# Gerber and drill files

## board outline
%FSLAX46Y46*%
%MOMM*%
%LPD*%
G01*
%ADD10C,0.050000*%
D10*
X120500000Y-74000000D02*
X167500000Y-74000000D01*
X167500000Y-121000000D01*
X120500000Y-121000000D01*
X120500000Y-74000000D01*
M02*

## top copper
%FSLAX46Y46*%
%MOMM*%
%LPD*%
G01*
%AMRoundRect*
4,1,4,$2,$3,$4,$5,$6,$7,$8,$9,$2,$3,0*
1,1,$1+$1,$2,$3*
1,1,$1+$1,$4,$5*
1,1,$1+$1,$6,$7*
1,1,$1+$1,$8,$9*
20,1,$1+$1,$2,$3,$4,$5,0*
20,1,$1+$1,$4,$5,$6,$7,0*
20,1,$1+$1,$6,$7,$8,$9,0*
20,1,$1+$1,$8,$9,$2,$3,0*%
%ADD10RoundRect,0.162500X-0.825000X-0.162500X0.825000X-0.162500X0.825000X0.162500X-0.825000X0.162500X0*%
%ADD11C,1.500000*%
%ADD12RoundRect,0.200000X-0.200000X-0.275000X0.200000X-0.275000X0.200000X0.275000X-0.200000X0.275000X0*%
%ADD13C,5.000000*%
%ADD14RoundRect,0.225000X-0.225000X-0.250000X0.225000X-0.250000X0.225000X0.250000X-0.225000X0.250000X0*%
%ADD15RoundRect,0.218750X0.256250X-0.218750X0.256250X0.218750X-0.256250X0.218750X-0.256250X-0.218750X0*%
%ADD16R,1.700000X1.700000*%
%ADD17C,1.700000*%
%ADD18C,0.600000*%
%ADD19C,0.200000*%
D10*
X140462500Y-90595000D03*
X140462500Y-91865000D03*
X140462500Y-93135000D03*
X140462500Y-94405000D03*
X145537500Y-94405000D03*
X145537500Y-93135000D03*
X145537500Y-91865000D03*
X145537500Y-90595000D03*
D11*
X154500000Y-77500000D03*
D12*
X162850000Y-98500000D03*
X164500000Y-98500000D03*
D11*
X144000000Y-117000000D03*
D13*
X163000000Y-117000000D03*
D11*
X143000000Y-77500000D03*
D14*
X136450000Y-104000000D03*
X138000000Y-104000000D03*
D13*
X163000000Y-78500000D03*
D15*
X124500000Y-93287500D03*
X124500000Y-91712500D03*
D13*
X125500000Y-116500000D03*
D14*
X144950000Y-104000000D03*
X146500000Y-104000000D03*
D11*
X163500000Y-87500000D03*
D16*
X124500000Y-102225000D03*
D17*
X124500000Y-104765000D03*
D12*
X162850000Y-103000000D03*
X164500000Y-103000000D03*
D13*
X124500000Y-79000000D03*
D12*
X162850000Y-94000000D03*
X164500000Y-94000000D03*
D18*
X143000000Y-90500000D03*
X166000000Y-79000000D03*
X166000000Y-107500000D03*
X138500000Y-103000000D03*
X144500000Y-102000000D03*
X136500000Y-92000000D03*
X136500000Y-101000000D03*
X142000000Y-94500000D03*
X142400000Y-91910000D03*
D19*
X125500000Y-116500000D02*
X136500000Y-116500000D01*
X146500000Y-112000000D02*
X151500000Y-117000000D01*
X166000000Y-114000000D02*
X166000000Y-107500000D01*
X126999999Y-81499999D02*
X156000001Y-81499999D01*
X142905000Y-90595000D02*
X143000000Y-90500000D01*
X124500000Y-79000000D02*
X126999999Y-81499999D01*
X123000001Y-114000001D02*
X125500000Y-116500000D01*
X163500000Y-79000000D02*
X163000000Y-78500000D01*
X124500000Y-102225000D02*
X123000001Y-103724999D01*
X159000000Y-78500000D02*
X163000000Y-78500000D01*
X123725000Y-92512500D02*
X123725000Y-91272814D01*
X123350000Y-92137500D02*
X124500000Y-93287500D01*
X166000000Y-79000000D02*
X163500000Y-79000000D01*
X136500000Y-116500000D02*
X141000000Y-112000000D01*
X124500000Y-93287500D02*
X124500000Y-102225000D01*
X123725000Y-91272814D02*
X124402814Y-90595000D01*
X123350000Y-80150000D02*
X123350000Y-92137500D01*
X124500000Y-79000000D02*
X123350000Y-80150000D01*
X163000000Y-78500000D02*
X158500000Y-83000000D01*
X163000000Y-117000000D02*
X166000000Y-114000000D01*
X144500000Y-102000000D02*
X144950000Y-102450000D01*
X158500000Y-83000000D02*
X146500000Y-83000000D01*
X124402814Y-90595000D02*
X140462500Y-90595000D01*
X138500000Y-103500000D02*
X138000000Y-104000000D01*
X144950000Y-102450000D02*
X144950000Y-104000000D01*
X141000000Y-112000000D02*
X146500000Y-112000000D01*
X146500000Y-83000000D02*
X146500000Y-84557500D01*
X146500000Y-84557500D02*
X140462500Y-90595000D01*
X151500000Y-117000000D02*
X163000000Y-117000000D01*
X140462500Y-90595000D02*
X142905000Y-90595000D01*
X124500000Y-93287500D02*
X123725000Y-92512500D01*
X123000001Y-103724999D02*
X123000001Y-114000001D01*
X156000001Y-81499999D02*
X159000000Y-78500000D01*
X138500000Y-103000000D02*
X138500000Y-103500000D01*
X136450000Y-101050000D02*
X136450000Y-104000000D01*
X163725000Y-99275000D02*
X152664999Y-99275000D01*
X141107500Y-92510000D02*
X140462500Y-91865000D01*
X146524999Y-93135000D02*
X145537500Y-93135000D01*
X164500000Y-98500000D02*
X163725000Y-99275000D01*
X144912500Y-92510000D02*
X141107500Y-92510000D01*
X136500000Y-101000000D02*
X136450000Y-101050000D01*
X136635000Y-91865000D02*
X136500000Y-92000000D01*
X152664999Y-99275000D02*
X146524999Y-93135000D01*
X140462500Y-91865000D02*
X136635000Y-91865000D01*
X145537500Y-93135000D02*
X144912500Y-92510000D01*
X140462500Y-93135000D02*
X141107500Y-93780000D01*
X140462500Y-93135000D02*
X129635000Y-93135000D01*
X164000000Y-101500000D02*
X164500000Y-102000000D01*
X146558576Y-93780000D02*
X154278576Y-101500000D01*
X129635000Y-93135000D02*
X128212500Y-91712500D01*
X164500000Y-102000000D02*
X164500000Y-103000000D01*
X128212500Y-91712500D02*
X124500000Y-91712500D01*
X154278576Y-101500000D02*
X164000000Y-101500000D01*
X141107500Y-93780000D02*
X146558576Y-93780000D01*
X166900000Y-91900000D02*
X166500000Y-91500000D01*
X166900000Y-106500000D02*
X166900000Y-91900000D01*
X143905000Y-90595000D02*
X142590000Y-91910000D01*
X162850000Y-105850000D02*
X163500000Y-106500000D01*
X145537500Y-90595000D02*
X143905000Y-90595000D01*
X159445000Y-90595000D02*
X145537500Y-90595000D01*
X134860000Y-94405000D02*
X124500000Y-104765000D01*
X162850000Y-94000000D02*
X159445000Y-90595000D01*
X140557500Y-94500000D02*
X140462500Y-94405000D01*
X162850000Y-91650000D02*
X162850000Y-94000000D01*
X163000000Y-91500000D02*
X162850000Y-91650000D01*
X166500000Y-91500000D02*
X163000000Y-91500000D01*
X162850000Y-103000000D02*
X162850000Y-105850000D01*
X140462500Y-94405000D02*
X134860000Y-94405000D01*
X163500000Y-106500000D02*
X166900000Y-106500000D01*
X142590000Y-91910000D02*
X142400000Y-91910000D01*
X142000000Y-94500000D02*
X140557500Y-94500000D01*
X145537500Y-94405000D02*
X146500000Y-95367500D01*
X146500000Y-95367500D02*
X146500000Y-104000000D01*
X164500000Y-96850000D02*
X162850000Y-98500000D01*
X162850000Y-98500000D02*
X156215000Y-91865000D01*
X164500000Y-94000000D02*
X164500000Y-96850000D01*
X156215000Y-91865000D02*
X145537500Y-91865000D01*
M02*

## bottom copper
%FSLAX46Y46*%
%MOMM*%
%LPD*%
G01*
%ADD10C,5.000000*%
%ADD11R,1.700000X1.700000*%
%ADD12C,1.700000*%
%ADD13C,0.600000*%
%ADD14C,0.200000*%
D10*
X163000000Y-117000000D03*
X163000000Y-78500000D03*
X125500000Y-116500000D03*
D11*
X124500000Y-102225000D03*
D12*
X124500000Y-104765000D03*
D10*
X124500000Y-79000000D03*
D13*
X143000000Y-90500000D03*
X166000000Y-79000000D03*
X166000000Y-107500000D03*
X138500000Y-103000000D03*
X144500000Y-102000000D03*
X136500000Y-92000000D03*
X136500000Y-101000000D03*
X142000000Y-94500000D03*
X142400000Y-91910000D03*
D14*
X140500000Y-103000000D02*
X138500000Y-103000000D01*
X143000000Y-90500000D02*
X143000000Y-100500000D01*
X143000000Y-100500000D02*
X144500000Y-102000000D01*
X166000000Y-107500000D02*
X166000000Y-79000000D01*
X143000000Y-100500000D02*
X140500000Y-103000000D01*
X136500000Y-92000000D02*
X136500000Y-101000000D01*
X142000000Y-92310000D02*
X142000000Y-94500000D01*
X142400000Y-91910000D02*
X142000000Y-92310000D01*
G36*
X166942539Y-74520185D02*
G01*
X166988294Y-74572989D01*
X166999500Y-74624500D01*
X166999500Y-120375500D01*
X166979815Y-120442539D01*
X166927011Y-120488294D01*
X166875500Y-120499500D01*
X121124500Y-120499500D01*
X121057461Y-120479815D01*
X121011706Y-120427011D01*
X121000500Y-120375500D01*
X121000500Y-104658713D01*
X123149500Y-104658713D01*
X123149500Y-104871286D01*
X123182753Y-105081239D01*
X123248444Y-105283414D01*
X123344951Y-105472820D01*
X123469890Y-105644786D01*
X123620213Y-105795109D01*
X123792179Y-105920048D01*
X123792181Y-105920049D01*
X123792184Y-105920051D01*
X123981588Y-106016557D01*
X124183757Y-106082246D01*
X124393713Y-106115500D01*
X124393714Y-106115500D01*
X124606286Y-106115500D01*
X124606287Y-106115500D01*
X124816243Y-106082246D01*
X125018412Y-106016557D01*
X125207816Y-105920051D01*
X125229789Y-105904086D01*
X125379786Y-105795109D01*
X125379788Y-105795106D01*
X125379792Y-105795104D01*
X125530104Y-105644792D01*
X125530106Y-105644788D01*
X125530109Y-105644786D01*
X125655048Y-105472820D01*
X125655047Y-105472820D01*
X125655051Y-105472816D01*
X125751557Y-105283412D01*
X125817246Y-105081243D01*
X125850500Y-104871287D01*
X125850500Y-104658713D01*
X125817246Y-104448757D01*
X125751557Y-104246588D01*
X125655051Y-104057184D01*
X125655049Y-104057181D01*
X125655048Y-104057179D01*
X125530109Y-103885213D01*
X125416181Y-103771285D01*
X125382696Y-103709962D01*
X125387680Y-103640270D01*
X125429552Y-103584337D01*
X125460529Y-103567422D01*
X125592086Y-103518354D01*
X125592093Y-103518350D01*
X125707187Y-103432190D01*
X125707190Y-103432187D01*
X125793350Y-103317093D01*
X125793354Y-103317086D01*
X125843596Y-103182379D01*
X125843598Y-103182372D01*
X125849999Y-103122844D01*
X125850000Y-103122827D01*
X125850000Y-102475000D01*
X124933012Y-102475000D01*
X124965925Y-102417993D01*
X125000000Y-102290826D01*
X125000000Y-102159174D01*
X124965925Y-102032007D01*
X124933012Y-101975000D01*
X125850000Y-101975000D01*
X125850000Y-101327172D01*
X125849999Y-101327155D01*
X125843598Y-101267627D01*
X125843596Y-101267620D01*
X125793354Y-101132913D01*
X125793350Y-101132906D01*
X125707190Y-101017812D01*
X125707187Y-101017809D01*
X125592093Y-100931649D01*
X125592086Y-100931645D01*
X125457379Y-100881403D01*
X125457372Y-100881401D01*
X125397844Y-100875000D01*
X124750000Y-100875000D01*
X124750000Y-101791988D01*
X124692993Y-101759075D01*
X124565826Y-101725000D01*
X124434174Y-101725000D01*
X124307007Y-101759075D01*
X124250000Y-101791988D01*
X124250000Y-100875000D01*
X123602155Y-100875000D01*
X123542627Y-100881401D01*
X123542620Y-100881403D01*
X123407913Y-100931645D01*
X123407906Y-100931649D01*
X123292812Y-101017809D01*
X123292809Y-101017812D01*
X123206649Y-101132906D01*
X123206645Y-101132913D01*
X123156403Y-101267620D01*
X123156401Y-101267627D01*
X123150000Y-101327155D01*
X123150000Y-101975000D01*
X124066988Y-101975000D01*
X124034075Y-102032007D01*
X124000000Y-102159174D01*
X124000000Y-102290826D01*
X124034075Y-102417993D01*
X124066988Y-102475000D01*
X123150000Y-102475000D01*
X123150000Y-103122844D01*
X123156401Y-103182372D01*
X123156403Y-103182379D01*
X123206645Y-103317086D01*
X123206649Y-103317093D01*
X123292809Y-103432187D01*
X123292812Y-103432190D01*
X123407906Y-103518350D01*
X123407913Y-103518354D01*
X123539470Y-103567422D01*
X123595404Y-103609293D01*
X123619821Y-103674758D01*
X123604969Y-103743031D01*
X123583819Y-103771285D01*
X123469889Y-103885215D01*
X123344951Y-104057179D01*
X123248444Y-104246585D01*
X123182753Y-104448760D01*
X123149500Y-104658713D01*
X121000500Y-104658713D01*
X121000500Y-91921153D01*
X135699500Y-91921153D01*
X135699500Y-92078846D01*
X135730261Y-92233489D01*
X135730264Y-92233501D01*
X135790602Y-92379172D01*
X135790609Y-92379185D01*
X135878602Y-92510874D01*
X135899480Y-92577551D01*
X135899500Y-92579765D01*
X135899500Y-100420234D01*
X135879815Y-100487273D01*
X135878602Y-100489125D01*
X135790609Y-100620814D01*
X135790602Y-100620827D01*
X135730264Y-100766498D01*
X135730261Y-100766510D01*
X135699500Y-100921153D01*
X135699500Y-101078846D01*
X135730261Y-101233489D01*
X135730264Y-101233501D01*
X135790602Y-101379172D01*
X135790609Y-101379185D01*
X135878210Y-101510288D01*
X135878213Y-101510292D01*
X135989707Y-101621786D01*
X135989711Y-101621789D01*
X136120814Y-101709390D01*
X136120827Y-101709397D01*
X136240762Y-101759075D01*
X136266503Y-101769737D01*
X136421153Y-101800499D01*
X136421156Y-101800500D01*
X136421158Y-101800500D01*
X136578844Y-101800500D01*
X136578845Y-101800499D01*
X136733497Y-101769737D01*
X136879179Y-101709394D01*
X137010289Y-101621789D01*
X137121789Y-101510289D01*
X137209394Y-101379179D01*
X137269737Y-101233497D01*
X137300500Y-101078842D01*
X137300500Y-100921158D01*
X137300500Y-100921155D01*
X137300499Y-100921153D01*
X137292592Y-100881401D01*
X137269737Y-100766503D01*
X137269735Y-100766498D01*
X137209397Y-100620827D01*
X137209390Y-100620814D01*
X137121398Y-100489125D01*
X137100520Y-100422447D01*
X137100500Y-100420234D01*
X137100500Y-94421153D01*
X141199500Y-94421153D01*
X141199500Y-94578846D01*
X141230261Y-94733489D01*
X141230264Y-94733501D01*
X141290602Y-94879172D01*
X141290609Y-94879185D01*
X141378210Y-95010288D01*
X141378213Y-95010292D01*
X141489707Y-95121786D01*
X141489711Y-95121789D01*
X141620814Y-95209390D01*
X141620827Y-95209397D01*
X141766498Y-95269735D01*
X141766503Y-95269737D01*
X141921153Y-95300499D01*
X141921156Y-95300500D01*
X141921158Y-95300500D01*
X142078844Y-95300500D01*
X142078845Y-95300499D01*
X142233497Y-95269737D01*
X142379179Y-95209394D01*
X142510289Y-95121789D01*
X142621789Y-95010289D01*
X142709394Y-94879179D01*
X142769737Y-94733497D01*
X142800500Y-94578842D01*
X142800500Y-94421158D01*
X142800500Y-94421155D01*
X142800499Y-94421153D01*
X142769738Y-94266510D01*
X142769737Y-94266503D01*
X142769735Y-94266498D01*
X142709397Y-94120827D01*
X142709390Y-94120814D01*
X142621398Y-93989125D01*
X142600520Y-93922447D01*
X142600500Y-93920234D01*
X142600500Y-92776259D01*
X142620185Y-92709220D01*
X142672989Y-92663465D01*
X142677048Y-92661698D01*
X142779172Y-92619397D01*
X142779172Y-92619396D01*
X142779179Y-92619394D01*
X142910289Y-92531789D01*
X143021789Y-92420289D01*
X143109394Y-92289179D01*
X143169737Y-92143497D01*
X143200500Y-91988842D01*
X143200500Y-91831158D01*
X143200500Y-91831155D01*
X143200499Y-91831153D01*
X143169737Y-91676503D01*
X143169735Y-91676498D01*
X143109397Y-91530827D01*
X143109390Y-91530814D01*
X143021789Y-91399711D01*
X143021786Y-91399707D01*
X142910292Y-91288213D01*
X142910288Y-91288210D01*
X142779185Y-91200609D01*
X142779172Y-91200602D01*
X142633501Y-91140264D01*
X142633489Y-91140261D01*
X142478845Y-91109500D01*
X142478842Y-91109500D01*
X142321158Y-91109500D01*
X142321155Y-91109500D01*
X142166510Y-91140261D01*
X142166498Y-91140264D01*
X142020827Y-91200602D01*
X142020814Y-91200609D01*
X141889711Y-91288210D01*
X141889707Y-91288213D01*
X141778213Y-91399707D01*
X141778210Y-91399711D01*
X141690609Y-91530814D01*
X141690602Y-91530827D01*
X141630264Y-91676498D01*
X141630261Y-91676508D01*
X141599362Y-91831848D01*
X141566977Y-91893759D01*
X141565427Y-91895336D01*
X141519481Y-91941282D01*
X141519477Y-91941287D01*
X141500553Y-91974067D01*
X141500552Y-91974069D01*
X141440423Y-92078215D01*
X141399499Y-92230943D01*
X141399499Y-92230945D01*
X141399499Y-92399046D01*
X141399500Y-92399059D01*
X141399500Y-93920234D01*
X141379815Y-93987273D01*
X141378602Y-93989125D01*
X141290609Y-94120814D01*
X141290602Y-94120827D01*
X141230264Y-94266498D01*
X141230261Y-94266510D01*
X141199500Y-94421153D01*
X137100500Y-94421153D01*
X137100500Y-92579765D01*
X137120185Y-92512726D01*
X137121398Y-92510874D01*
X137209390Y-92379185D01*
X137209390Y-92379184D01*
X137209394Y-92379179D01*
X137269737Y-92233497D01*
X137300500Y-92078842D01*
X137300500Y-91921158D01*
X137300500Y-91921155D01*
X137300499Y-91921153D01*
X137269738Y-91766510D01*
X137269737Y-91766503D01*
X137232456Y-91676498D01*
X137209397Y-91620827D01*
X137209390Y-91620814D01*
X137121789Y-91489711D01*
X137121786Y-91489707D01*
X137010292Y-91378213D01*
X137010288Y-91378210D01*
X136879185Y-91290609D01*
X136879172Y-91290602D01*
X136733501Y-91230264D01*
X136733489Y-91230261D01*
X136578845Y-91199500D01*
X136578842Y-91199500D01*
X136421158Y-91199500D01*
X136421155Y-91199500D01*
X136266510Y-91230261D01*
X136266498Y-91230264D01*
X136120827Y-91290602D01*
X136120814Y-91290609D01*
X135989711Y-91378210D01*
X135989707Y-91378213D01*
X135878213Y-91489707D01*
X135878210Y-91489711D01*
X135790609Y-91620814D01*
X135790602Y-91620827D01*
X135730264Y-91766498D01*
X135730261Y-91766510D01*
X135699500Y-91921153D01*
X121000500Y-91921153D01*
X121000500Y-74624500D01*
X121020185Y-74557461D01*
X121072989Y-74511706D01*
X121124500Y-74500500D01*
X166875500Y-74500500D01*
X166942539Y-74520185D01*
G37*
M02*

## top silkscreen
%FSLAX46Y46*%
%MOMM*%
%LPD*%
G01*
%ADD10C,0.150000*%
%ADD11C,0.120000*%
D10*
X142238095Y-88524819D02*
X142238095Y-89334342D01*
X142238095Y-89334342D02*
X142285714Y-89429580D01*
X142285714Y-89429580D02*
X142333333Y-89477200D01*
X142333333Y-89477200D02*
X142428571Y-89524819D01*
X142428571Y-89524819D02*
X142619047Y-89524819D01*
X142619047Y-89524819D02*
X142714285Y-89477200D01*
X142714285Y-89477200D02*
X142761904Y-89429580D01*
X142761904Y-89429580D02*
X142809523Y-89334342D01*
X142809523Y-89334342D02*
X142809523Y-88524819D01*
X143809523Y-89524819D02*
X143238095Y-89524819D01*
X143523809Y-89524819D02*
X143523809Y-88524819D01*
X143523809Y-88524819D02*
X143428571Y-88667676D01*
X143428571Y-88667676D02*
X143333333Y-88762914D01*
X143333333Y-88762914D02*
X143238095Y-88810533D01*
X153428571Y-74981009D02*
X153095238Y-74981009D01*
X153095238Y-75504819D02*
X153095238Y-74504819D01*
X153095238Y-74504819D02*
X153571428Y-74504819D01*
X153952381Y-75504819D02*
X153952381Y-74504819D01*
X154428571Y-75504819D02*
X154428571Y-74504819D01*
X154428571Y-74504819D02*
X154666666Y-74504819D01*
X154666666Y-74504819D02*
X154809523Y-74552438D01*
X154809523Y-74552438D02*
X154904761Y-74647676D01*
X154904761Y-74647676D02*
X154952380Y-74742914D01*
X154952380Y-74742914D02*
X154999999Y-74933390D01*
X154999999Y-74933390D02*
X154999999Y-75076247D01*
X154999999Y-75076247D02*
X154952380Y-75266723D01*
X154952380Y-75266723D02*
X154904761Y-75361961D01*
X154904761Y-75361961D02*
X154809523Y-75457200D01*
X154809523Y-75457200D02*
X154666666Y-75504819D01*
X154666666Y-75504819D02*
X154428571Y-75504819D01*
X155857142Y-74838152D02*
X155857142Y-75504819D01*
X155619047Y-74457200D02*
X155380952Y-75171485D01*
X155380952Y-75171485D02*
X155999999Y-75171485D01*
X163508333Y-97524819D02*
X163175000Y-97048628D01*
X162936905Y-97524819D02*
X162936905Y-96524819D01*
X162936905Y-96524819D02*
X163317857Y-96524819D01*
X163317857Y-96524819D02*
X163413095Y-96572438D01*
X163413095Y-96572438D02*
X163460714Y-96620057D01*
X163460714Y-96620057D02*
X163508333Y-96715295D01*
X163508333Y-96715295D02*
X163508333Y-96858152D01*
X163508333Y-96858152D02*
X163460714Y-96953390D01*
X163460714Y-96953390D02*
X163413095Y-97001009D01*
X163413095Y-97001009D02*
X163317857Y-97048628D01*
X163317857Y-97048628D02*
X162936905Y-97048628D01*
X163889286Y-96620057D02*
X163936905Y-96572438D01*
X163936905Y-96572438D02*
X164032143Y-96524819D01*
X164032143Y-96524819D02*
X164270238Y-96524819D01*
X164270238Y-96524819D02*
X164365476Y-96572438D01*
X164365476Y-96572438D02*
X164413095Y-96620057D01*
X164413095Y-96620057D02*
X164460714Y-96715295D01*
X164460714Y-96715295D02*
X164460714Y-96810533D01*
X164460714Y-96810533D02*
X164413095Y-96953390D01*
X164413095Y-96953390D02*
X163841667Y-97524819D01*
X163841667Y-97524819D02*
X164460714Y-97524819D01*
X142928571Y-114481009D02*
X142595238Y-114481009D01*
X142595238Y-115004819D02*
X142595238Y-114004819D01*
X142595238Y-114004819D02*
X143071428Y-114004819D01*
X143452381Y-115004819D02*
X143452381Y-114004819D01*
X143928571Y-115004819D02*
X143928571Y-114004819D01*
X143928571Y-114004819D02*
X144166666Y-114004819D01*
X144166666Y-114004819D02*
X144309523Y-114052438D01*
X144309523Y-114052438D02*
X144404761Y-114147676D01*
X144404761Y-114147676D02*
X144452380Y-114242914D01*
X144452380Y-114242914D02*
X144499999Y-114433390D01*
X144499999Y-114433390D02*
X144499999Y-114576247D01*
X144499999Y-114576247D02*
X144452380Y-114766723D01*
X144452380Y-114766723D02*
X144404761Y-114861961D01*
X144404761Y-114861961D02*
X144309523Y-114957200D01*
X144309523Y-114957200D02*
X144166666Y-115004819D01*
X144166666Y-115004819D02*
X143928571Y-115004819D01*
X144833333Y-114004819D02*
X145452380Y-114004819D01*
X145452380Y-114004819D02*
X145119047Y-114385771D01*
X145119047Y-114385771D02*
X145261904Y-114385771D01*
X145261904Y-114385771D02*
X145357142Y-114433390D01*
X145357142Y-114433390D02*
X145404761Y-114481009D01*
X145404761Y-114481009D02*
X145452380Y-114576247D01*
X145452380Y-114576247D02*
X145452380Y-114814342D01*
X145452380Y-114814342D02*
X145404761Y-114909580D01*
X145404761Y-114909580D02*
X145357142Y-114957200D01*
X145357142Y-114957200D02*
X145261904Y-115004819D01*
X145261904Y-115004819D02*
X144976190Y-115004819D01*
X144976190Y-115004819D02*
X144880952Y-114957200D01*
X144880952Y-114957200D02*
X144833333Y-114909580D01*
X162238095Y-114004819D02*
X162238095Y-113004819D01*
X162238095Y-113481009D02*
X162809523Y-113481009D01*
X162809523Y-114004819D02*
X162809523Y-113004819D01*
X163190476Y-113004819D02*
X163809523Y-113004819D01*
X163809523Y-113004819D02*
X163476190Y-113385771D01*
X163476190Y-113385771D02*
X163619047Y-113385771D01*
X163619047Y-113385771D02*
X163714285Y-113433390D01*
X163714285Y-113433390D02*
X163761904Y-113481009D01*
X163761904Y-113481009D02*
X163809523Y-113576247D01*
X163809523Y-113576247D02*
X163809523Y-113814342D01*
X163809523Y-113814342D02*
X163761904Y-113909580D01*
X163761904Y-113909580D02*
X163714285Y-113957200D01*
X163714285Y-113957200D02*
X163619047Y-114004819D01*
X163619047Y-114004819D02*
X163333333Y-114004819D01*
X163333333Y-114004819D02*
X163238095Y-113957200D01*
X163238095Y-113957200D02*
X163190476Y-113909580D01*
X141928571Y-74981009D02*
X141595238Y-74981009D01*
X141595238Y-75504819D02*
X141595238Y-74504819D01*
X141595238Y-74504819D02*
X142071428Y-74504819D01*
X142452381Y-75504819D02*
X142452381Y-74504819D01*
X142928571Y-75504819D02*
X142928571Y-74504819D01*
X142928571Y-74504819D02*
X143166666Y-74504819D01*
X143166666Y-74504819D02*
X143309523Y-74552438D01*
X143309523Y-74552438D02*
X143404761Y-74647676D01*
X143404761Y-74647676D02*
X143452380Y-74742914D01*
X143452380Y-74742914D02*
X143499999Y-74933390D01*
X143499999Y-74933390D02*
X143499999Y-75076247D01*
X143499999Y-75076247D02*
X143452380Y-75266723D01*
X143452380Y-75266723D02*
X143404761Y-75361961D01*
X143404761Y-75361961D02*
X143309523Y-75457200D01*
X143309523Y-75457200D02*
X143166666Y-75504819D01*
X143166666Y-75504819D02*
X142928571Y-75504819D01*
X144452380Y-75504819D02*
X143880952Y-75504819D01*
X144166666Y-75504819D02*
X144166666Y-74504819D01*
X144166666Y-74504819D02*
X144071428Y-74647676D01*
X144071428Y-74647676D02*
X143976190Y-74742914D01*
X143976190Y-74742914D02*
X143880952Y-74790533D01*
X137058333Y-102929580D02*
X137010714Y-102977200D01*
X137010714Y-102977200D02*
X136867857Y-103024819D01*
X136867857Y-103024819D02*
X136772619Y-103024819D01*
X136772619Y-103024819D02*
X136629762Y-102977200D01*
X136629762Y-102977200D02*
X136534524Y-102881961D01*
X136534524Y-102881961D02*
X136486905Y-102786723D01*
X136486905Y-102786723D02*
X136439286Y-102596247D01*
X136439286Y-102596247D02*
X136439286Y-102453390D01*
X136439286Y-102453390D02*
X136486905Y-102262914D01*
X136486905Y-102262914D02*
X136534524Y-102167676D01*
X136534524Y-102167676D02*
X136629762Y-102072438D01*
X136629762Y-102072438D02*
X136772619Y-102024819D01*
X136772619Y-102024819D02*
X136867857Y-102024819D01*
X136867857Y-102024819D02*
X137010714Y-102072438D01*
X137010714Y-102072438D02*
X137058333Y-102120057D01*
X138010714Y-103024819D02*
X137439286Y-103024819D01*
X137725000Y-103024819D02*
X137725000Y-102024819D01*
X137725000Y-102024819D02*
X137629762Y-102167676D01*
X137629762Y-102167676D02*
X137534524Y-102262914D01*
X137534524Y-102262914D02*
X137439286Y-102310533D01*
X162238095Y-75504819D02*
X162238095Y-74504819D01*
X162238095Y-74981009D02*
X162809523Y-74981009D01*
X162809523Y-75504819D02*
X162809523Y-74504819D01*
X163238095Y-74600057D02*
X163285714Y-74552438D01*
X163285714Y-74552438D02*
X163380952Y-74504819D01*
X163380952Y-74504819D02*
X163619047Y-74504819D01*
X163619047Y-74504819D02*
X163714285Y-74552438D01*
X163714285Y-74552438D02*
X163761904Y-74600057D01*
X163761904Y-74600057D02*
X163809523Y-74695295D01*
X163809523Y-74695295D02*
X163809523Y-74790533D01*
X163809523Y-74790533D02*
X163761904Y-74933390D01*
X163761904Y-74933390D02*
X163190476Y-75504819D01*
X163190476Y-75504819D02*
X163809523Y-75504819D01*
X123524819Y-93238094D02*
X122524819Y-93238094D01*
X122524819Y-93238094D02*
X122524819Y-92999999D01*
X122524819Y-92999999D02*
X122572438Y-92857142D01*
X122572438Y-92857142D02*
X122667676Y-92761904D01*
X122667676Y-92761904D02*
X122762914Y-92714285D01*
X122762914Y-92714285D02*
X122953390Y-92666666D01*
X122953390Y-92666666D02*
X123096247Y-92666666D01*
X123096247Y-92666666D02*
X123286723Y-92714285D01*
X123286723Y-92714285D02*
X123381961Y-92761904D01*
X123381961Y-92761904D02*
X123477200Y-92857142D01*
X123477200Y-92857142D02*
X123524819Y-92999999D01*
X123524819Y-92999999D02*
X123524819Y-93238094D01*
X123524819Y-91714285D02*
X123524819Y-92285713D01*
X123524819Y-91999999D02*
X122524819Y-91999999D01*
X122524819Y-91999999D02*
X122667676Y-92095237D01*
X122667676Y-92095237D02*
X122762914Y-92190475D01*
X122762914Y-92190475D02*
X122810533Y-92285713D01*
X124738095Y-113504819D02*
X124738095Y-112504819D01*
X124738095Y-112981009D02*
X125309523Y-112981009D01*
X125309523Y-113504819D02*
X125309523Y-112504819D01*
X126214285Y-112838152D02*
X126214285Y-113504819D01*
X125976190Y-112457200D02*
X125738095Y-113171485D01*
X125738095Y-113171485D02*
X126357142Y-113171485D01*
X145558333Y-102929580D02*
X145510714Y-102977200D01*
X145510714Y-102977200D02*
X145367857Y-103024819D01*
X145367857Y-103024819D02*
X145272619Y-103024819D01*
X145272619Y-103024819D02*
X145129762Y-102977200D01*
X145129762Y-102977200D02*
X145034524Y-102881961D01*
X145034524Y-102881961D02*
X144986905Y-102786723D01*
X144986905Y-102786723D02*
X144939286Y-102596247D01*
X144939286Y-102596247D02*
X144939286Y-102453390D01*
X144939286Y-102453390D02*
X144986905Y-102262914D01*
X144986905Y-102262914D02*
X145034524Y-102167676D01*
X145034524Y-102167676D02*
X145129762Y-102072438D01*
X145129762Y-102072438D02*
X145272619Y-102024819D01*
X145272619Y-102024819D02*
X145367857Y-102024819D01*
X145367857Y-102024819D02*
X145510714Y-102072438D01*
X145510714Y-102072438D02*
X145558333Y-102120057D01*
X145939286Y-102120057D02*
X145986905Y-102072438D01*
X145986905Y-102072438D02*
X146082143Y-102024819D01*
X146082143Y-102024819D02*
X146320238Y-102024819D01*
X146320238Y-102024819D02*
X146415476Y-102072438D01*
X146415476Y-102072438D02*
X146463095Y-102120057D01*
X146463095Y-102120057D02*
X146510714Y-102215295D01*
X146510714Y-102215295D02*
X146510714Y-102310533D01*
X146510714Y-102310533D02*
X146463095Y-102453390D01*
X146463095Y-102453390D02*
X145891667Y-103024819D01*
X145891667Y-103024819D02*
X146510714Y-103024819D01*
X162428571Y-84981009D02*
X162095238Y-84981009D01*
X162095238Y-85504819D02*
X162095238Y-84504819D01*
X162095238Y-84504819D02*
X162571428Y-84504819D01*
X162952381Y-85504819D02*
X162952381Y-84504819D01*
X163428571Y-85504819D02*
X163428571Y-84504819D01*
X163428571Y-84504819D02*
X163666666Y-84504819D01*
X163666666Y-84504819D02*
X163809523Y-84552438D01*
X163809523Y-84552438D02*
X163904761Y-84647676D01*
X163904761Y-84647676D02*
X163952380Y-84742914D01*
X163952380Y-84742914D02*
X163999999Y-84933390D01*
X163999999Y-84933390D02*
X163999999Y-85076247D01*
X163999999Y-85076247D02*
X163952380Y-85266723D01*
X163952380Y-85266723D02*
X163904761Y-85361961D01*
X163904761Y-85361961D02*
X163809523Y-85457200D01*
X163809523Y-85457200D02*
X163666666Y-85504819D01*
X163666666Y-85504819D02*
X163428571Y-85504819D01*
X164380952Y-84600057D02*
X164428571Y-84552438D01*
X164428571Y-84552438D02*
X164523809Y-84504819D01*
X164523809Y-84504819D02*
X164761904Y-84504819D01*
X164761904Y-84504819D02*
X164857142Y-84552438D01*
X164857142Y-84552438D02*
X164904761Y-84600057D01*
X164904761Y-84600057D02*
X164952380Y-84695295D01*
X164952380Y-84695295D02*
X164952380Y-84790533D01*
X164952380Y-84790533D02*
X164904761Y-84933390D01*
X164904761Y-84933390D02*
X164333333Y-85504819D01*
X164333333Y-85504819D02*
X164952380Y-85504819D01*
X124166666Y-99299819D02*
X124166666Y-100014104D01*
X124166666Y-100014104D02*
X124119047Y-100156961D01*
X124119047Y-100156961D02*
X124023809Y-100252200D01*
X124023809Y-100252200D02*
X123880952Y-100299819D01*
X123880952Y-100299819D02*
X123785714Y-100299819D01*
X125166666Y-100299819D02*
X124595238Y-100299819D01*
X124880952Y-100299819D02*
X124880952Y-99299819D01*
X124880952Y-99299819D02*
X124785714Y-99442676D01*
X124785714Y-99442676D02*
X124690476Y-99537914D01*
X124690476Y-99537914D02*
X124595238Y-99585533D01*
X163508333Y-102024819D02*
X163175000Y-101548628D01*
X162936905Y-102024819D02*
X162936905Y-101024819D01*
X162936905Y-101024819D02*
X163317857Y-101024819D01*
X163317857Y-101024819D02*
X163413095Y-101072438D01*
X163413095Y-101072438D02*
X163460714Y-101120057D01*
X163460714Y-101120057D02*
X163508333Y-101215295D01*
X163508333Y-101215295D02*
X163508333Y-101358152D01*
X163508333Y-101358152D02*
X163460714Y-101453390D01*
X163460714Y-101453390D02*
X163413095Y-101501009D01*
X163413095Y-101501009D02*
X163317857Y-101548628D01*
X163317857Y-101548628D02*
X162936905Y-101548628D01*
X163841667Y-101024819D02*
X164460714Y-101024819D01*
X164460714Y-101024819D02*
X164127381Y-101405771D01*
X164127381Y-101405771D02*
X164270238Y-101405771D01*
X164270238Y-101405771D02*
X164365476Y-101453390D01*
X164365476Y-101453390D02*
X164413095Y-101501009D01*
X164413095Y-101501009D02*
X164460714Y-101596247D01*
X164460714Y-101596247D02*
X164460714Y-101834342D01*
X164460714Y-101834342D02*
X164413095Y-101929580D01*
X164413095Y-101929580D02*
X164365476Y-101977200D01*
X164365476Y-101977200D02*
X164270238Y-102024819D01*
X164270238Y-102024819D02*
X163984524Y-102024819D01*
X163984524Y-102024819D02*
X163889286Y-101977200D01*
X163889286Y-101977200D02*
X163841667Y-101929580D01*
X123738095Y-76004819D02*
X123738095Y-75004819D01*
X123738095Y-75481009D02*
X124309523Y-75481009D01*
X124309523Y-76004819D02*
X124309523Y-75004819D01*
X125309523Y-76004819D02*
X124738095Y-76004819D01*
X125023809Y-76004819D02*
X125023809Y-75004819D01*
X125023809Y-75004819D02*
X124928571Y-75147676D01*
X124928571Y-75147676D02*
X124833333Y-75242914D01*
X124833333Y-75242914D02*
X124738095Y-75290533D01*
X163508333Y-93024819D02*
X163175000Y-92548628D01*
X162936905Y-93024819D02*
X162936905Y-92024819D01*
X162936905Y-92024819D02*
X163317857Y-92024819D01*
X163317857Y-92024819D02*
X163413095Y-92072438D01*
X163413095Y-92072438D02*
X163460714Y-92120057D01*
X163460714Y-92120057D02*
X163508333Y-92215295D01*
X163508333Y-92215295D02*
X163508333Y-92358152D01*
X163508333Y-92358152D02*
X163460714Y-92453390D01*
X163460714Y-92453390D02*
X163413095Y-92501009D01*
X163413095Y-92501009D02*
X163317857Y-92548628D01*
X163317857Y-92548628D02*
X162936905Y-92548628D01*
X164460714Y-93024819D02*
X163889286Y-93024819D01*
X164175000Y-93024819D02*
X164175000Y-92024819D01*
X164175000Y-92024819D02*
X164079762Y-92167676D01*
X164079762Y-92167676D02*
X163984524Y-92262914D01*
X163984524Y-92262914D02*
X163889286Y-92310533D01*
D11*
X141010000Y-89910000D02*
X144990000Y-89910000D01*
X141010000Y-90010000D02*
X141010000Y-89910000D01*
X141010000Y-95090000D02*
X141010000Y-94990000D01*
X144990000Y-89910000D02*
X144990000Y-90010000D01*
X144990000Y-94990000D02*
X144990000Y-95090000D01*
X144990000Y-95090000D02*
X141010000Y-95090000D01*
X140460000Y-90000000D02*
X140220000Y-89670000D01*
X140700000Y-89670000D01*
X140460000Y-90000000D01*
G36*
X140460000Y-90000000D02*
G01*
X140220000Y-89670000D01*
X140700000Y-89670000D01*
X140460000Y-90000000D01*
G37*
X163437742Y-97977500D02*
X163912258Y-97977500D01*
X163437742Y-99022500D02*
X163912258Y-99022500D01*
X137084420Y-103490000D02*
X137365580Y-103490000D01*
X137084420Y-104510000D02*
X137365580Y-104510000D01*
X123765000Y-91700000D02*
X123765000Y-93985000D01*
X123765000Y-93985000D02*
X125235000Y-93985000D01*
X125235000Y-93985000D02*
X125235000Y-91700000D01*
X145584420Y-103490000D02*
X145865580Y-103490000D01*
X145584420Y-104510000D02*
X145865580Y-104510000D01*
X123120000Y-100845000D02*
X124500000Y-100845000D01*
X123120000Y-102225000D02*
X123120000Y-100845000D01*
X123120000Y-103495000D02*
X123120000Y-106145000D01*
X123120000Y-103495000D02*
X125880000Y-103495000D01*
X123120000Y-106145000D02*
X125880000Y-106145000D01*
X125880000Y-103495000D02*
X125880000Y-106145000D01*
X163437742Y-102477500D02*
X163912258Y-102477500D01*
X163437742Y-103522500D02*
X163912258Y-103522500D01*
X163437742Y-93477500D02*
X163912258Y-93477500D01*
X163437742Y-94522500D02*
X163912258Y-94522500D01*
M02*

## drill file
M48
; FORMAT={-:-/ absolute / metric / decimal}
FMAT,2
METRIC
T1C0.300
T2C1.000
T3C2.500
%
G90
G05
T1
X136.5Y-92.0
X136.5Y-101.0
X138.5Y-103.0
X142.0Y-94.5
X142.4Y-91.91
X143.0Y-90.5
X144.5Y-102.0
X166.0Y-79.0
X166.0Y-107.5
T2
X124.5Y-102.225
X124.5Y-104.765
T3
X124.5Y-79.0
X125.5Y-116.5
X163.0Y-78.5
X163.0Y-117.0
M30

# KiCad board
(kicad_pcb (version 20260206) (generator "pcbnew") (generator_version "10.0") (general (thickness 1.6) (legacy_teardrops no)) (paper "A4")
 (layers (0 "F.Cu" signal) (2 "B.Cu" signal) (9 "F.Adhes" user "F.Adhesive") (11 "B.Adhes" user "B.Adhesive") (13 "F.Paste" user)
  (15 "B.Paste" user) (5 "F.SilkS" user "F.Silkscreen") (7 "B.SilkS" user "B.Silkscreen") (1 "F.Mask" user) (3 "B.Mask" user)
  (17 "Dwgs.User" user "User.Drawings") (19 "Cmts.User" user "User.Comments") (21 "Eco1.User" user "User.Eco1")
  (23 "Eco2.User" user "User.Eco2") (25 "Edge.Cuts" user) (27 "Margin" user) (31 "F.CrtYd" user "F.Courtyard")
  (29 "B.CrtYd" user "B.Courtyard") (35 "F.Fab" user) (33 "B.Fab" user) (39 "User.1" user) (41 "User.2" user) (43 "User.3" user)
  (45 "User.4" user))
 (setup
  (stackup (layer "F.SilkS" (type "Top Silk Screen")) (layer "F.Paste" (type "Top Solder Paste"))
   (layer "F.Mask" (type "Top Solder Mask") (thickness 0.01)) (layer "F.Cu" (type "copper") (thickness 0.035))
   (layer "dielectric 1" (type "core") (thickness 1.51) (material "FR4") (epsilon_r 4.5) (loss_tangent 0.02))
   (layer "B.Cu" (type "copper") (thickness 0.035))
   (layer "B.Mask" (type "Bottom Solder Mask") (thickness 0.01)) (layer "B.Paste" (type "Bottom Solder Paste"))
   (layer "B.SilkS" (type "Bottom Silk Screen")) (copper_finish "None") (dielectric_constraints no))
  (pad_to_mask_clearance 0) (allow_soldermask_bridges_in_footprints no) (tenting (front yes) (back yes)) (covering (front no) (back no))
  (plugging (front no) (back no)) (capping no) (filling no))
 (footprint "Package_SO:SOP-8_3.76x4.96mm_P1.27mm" (layer "F.Cu") (at 143 92.5)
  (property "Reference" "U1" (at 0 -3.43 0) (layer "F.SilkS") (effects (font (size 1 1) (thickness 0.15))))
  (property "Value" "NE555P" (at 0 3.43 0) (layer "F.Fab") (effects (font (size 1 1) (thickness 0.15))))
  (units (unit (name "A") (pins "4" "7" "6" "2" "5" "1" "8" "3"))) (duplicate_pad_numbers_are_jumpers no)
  (fp_line (start -1.99 -2.59) (end 1.99 -2.59) (stroke (width 0.12) (type solid)) (layer "F.SilkS"))
  (fp_line (start -1.99 -2.49) (end -1.99 -2.59) (stroke (width 0.12) (type solid)) (layer "F.SilkS"))
  (fp_line (start -1.99 2.59) (end -1.99 2.49) (stroke (width 0.12) (type solid)) (layer "F.SilkS"))
  (fp_line (start 1.99 -2.59) (end 1.99 -2.49) (stroke (width 0.12) (type solid)) (layer "F.SilkS"))
  (fp_line (start 1.99 2.49) (end 1.99 2.59) (stroke (width 0.12) (type solid)) (layer "F.SilkS"))
  (fp_line (start 1.99 2.59) (end -1.99 2.59) (stroke (width 0.12) (type solid)) (layer "F.SilkS"))
  (fp_poly (pts (xy -2.54 -2.5) (xy -2.78 -2.83) (xy -2.3 -2.83)) (stroke (width 0.12) (type solid)) (fill yes) (layer "F.SilkS"))
  (pad "1" smd roundrect (at -2.5375 -1.905) (size 1.975 0.65) (layers "F.Cu" "F.Mask" "F.Paste") (roundrect_rratio 0.25) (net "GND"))
  (pad "2" smd roundrect (at -2.5375 -0.635) (size 1.975 0.65) (layers "F.Cu" "F.Mask" "F.Paste") (roundrect_rratio 0.25) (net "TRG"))
  (pad "3" smd roundrect (at -2.5375 0.635) (size 1.975 0.65) (layers "F.Cu" "F.Mask" "F.Paste") (roundrect_rratio 0.25) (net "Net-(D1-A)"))
  (pad "4" smd roundrect (at -2.5375 1.905) (size 1.975 0.65) (layers "F.Cu" "F.Mask" "F.Paste") (roundrect_rratio 0.25) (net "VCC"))
  (pad "5" smd roundrect (at 2.5375 1.905) (size 1.975 0.65) (layers "F.Cu" "F.Mask" "F.Paste") (roundrect_rratio 0.25)
   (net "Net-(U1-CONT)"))
  (pad "6" smd roundrect (at 2.5375 0.635) (size 1.975 0.65) (layers "F.Cu" "F.Mask" "F.Paste") (roundrect_rratio 0.25) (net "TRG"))
  (pad "7" smd roundrect (at 2.5375 -0.635) (size 1.975 0.65) (layers "F.Cu" "F.Mask" "F.Paste") (roundrect_rratio 0.25) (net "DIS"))
  (pad "8" smd roundrect (at 2.5375 -1.905) (size 1.975 0.65) (layers "F.Cu" "F.Mask" "F.Paste") (roundrect_rratio 0.25) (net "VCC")))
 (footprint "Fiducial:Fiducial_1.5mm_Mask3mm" (layer "F.Cu") (at 154.5 77.5)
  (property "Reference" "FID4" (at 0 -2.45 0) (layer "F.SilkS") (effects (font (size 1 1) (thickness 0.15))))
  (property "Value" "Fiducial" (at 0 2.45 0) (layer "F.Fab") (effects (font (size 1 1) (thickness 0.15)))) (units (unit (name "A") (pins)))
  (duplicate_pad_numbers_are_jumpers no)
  (pad "" smd circle (at 0 0) (size 1.5 1.5) (layers "F.Cu" "F.Mask") (solder_mask_margin 0.75) (clearance 0.85)))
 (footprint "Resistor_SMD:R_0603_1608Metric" (layer "F.Cu") (at 163.675 98.5)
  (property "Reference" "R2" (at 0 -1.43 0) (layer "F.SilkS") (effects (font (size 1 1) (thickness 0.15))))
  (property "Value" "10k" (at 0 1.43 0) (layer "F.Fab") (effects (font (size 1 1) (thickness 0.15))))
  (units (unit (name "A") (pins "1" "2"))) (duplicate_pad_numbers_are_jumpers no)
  (fp_line (start -0.237258 -0.5225) (end 0.237258 -0.5225) (stroke (width 0.12) (type solid)) (layer "F.SilkS"))
  (fp_line (start -0.237258 0.5225) (end 0.237258 0.5225) (stroke (width 0.12) (type solid)) (layer "F.SilkS"))
  (pad "1" smd roundrect (at -0.825 0) (size 0.8 0.95) (layers "F.Cu" "F.Mask" "F.Paste") (roundrect_rratio 0.25) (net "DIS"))
  (pad "2" smd roundrect (at 0.825 0) (size 0.8 0.95) (layers "F.Cu" "F.Mask" "F.Paste") (roundrect_rratio 0.25) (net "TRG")))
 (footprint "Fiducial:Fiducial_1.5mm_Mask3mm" (layer "F.Cu") (at 144 117)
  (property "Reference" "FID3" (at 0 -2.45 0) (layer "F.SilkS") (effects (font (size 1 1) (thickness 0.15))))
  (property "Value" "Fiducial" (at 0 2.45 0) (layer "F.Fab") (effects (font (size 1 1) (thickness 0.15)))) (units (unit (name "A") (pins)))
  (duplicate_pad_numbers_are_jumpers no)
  (pad "" smd circle (at 0 0) (size 1.5 1.5) (layers "F.Cu" "F.Mask") (solder_mask_margin 0.75) (clearance 0.85)))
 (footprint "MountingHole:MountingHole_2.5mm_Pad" (layer "F.Cu") (at 163 117)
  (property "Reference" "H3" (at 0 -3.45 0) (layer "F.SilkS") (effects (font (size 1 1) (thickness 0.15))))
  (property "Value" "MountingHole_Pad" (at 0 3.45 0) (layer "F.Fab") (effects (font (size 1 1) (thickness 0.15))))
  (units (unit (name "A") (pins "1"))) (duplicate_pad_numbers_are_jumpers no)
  (pad "1" thru_hole circle (at 0 0) (size 5 5) (drill 2.5) (layers "*.Cu" "*.Mask") (remove_unused_layers no) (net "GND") (zone_connect 2)))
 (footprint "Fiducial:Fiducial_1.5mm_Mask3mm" (layer "F.Cu") (at 143 77.5)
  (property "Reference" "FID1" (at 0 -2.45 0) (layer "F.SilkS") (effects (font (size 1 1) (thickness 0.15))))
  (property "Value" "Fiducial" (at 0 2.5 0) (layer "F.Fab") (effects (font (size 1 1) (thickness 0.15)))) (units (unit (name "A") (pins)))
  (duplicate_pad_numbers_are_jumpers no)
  (pad "" smd circle (at 0 0) (size 1.5 1.5) (layers "F.Cu" "F.Mask") (solder_mask_margin 0.75) (clearance 0.85)))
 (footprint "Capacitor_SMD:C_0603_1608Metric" (layer "F.Cu") (at 137.225 104)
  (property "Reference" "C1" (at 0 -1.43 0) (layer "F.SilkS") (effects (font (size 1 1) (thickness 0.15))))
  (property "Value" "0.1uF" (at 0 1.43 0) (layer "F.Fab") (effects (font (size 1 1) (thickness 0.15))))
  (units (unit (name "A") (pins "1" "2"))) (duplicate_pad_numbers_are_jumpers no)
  (fp_line (start -0.14058 -0.51) (end 0.14058 -0.51) (stroke (width 0.12) (type solid)) (layer "F.SilkS"))
  (fp_line (start -0.14058 0.51) (end 0.14058 0.51) (stroke (width 0.12) (type solid)) (layer "F.SilkS"))
  (pad "1" smd roundrect (at -0.775 0) (size 0.9 0.95) (layers "F.Cu" "F.Mask" "F.Paste") (roundrect_rratio 0.25) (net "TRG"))
  (pad "2" smd roundrect (at 0.775 0) (size 0.9 0.95) (layers "F.Cu" "F.Mask" "F.Paste") (roundrect_rratio 0.25) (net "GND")))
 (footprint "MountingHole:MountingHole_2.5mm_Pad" (layer "F.Cu") (at 163 78.5)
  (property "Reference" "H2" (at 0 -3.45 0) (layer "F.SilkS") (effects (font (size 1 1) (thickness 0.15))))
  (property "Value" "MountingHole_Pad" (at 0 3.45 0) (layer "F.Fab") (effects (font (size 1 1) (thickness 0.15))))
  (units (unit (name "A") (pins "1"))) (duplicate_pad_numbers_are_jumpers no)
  (pad "1" thru_hole circle (at 0 0) (size 5 5) (drill 2.5) (layers "*.Cu" "*.Mask") (remove_unused_layers no) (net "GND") (zone_connect 2)))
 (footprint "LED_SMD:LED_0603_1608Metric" (layer "F.Cu") (at 124.5 92.5 90)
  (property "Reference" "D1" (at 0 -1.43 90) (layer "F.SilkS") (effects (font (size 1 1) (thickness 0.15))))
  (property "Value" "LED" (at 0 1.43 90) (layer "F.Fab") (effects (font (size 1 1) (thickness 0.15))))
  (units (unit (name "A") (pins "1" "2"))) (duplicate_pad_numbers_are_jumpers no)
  (fp_line (start 0.8 -0.735) (end -1.485 -0.735) (stroke (width 0.12) (type solid)) (layer "F.SilkS"))
  (fp_line (start -1.485 -0.735) (end -1.485 0.735) (stroke (width 0.12) (type solid)) (layer "F.SilkS"))
  (fp_line (start -1.485 0.735) (end 0.8 0.735) (stroke (width 0.12) (type solid)) (layer "F.SilkS"))
  (pad "1" smd roundrect (at -0.7875 0 90) (size 0.875 0.95) (layers "F.Cu" "F.Mask" "F.Paste") (roundrect_rratio 0.25) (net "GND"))
  (pad "2" smd roundrect (at 0.7875 0 90) (size 0.875 0.95) (layers "F.Cu" "F.Mask" "F.Paste") (roundrect_rratio 0.25) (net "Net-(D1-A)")))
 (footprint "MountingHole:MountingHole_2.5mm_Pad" (layer "F.Cu") (at 125.5 116.5)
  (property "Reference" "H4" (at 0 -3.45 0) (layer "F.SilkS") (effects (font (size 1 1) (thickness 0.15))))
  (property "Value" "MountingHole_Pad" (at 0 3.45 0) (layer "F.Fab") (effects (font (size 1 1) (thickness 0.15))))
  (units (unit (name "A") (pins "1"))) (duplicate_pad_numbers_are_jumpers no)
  (pad "1" thru_hole circle (at 0 0) (size 5 5) (drill 2.5) (layers "*.Cu" "*.Mask") (remove_unused_layers no) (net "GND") (zone_connect 2)))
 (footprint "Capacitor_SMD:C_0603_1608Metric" (layer "F.Cu") (at 145.725 104)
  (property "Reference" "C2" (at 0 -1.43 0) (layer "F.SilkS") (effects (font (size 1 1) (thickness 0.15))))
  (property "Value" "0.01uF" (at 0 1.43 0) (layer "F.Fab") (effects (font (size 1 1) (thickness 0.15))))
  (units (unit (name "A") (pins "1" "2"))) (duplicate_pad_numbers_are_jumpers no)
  (fp_line (start -0.14058 -0.51) (end 0.14058 -0.51) (stroke (width 0.12) (type solid)) (layer "F.SilkS"))
  (fp_line (start -0.14058 0.51) (end 0.14058 0.51) (stroke (width 0.12) (type solid)) (layer "F.SilkS"))
  (pad "1" smd roundrect (at -0.775 0) (size 0.9 0.95) (layers "F.Cu" "F.Mask" "F.Paste") (roundrect_rratio 0.25) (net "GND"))
  (pad "2" smd roundrect (at 0.775 0) (size 0.9 0.95) (layers "F.Cu" "F.Mask" "F.Paste") (roundrect_rratio 0.25) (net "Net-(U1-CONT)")))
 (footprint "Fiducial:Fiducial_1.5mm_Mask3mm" (layer "F.Cu") (at 163.5 87.5)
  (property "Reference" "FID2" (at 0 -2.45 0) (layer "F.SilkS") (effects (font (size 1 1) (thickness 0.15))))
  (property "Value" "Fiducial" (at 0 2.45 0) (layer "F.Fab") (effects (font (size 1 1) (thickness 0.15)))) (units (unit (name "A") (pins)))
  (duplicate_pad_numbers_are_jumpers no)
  (pad "" smd circle (at 0 0) (size 1.5 1.5) (layers "F.Cu" "F.Mask") (solder_mask_margin 0.75) (clearance 0.85)))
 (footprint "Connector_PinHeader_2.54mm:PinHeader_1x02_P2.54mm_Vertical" (layer "F.Cu") (at 124.5 102.225)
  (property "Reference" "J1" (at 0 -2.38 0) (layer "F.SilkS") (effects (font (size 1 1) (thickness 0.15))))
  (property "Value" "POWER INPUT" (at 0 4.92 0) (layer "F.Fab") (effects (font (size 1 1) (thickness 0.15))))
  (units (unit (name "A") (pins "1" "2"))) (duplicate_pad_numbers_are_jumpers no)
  (fp_line (start -1.38 -1.38) (end 0 -1.38) (stroke (width 0.12) (type solid)) (layer "F.SilkS"))
  (fp_line (start -1.38 0) (end -1.38 -1.38) (stroke (width 0.12) (type solid)) (layer "F.SilkS"))
  (fp_line (start -1.38 1.27) (end -1.38 3.92) (stroke (width 0.12) (type solid)) (layer "F.SilkS"))
  (fp_line (start -1.38 1.27) (end 1.38 1.27) (stroke (width 0.12) (type solid)) (layer "F.SilkS"))
  (fp_line (start -1.38 3.92) (end 1.38 3.92) (stroke (width 0.12) (type solid)) (layer "F.SilkS"))
  (fp_line (start 1.38 1.27) (end 1.38 3.92) (stroke (width 0.12) (type solid)) (layer "F.SilkS"))
  (pad "1" thru_hole rect (at 0 0) (size 1.7 1.7) (drill 1) (layers "*.Cu" "*.Mask") (remove_unused_layers no) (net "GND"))
  (pad "2" thru_hole circle (at 0 2.54) (size 1.7 1.7) (drill 1) (layers "*.Cu" "*.Mask") (remove_unused_layers no) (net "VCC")))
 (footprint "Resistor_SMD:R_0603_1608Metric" (layer "F.Cu") (at 163.675 103)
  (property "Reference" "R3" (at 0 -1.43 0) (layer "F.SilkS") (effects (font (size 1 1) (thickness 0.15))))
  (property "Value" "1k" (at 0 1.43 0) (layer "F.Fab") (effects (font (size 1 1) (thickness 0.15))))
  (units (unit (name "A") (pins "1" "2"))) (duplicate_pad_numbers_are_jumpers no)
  (fp_line (start -0.237258 -0.5225) (end 0.237258 -0.5225) (stroke (width 0.12) (type solid)) (layer "F.SilkS"))
  (fp_line (start -0.237258 0.5225) (end 0.237258 0.5225) (stroke (width 0.12) (type solid)) (layer "F.SilkS"))
  (pad "1" smd roundrect (at -0.825 0) (size 0.8 0.95) (layers "F.Cu" "F.Mask" "F.Paste") (roundrect_rratio 0.25) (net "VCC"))
  (pad "2" smd roundrect (at 0.825 0) (size 0.8 0.95) (layers "F.Cu" "F.Mask" "F.Paste") (roundrect_rratio 0.25) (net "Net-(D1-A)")))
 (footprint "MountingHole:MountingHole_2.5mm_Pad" (layer "F.Cu") (at 124.5 79)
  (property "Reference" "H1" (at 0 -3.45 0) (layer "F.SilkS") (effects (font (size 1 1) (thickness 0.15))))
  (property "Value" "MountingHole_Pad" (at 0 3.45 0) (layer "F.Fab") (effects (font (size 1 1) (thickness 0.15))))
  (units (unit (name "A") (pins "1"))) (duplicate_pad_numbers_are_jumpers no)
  (pad "1" thru_hole circle (at 0 0) (size 5 5) (drill 2.5) (layers "*.Cu" "*.Mask") (remove_unused_layers no) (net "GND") (zone_connect 2)))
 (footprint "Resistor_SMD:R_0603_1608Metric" (layer "F.Cu") (at 163.675 94)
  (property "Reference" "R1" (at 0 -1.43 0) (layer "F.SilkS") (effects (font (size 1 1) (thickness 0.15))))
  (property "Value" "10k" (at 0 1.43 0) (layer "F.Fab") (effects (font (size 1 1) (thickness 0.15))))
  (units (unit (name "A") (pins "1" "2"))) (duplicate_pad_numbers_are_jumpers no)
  (fp_line (start -0.237258 -0.5225) (end 0.237258 -0.5225) (stroke (width 0.12) (type solid)) (layer "F.SilkS"))
  (fp_line (start -0.237258 0.5225) (end 0.237258 0.5225) (stroke (width 0.12) (type solid)) (layer "F.SilkS"))
  (pad "1" smd roundrect (at -0.825 0) (size 0.8 0.95) (layers "F.Cu" "F.Mask" "F.Paste") (roundrect_rratio 0.25) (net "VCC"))
  (pad "2" smd roundrect (at 0.825 0) (size 0.8 0.95) (layers "F.Cu" "F.Mask" "F.Paste") (roundrect_rratio 0.25) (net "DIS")))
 (gr_rect (start 120.5 74) (end 167.5 121) (stroke (width 0.05) (type default)) (fill no) (layer "Edge.Cuts"))
 (segment (start 125.5 116.5) (end 136.5 116.5) (width 0.2) (layer "F.Cu") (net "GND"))
 (segment (start 146.5 112) (end 151.5 117) (width 0.2) (layer "F.Cu") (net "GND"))
 (segment (start 166 114) (end 166 107.5) (width 0.2) (layer "F.Cu") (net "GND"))
 (segment (start 126.999999 81.499999) (end 156.000001 81.499999) (width 0.2) (layer "F.Cu") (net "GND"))
 (segment (start 142.905 90.595) (end 143 90.5) (width 0.2) (layer "F.Cu") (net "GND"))
 (segment (start 124.5 79) (end 126.999999 81.499999) (width 0.2) (layer "F.Cu") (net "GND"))
 (segment (start 123.000001 114.000001) (end 125.5 116.5) (width 0.2) (layer "F.Cu") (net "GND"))
 (segment (start 163.5 79) (end 163 78.5) (width 0.2) (layer "F.Cu") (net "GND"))
 (segment (start 124.5 102.225) (end 123.000001 103.724999) (width 0.2) (layer "F.Cu") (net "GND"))
 (segment (start 159 78.5) (end 163 78.5) (width 0.2) (layer "F.Cu") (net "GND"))
 (segment (start 123.725 92.5125) (end 123.725 91.272814) (width 0.2) (layer "F.Cu") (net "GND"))
 (segment (start 123.35 92.1375) (end 124.5 93.2875) (width 0.2) (layer "F.Cu") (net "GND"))
 (segment (start 166 79) (end 163.5 79) (width 0.2) (layer "F.Cu") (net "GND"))
 (segment (start 136.5 116.5) (end 141 112) (width 0.2) (layer "F.Cu") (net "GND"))
 (segment (start 124.5 93.2875) (end 124.5 102.225) (width 0.2) (layer "F.Cu") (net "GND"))
 (segment (start 123.725 91.272814) (end 124.402814 90.595) (width 0.2) (layer "F.Cu") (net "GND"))
 (segment (start 123.35 80.15) (end 123.35 92.1375) (width 0.2) (layer "F.Cu") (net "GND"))
 (segment (start 124.5 79) (end 123.35 80.15) (width 0.2) (layer "F.Cu") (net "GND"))
 (segment (start 163 78.5) (end 158.5 83) (width 0.2) (layer "F.Cu") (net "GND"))
 (segment (start 163 117) (end 166 114) (width 0.2) (layer "F.Cu") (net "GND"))
 (segment (start 144.5 102) (end 144.95 102.45) (width 0.2) (layer "F.Cu") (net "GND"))
 (segment (start 158.5 83) (end 146.5 83) (width 0.2) (layer "F.Cu") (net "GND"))
 (segment (start 124.402814 90.595) (end 140.4625 90.595) (width 0.2) (layer "F.Cu") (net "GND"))
 (segment (start 138.5 103.5) (end 138 104) (width 0.2) (layer "F.Cu") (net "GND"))
 (segment (start 144.95 102.45) (end 144.95 104) (width 0.2) (layer "F.Cu") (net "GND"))
 (segment (start 141 112) (end 146.5 112) (width 0.2) (layer "F.Cu") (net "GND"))
 (segment (start 146.5 83) (end 146.5 84.5575) (width 0.2) (layer "F.Cu") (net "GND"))
 (segment (start 146.5 84.5575) (end 140.4625 90.595) (width 0.2) (layer "F.Cu") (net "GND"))
 (segment (start 151.5 117) (end 163 117) (width 0.2) (layer "F.Cu") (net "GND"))
 (segment (start 140.4625 90.595) (end 142.905 90.595) (width 0.2) (layer "F.Cu") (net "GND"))
 (segment (start 124.5 93.2875) (end 123.725 92.5125) (width 0.2) (layer "F.Cu") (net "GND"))
 (segment (start 123.000001 103.724999) (end 123.000001 114.000001) (width 0.2) (layer "F.Cu") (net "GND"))
 (segment (start 156.000001 81.499999) (end 159 78.5) (width 0.2) (layer "F.Cu") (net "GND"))
 (segment (start 138.5 103) (end 138.5 103.5) (width 0.2) (layer "F.Cu") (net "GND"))
 (via (at 143 90.5) (size 0.6) (drill 0.3) (layers "F.Cu" "B.Cu") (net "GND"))
 (via (at 166 79) (size 0.6) (drill 0.3) (layers "F.Cu" "B.Cu") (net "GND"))
 (via (at 166 107.5) (size 0.6) (drill 0.3) (layers "F.Cu" "B.Cu") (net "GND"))
 (via (at 138.5 103) (size 0.6) (drill 0.3) (layers "F.Cu" "B.Cu") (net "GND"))
 (via (at 144.5 102) (size 0.6) (drill 0.3) (layers "F.Cu" "B.Cu") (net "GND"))
 (segment (start 140.5 103) (end 138.5 103) (width 0.2) (layer "B.Cu") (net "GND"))
 (segment (start 143 90.5) (end 143 100.5) (width 0.2) (layer "B.Cu") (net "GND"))
 (segment (start 143 100.5) (end 144.5 102) (width 0.2) (layer "B.Cu") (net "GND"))
 (segment (start 166 107.5) (end 166 79) (width 0.2) (layer "B.Cu") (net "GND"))
 (segment (start 143 100.5) (end 140.5 103) (width 0.2) (layer "B.Cu") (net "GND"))
 (segment (start 136.45 101.05) (end 136.45 104) (width 0.2) (layer "F.Cu") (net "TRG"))
 (segment (start 163.725 99.275) (end 152.664999 99.275) (width 0.2) (layer "F.Cu") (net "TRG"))
 (segment (start 141.1075 92.51) (end 140.4625 91.865) (width 0.2) (layer "F.Cu") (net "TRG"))
 (segment (start 146.524999 93.135) (end 145.5375 93.135) (width 0.2) (layer "F.Cu") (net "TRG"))
 (segment (start 164.5 98.5) (end 163.725 99.275) (width 0.2) (layer "F.Cu") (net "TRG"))
 (segment (start 144.9125 92.51) (end 141.1075 92.51) (width 0.2) (layer "F.Cu") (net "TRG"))
 (segment (start 136.5 101) (end 136.45 101.05) (width 0.2) (layer "F.Cu") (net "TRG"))
 (segment (start 136.635 91.865) (end 136.5 92) (width 0.2) (layer "F.Cu") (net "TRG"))
 (segment (start 152.664999 99.275) (end 146.524999 93.135) (width 0.2) (layer "F.Cu") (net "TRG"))
 (segment (start 140.4625 91.865) (end 136.635 91.865) (width 0.2) (layer "F.Cu") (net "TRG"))
 (segment (start 145.5375 93.135) (end 144.9125 92.51) (width 0.2) (layer "F.Cu") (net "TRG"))
 (via (at 136.5 92) (size 0.6) (drill 0.3) (layers "F.Cu" "B.Cu") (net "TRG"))
 (via (at 136.5 101) (size 0.6) (drill 0.3) (layers "F.Cu" "B.Cu") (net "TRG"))
 (segment (start 136.5 92) (end 136.5 101) (width 0.2) (layer "B.Cu") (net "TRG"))
 (segment (start 140.4625 93.135) (end 141.1075 93.78) (width 0.2) (layer "F.Cu") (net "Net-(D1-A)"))
 (segment (start 140.4625 93.135) (end 129.635 93.135) (width 0.2) (layer "F.Cu") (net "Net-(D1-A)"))
 (segment (start 164 101.5) (end 164.5 102) (width 0.2) (layer "F.Cu") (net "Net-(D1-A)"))
 (segment (start 146.558576 93.78) (end 154.278576 101.5) (width 0.2) (layer "F.Cu") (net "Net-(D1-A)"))
 (segment (start 129.635 93.135) (end 128.2125 91.7125) (width 0.2) (layer "F.Cu") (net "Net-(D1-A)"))
 (segment (start 164.5 102) (end 164.5 103) (width 0.2) (layer "F.Cu") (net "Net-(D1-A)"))
 (segment (start 128.2125 91.7125) (end 124.5 91.7125) (width 0.2) (layer "F.Cu") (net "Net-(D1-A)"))
 (segment (start 154.278576 101.5) (end 164 101.5) (width 0.2) (layer "F.Cu") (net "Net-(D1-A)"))
 (segment (start 141.1075 93.78) (end 146.558576 93.78) (width 0.2) (layer "F.Cu") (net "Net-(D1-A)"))
 (segment (start 166.9 91.9) (end 166.5 91.5) (width 0.2) (layer "F.Cu") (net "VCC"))
 (segment (start 166.9 106.5) (end 166.9 91.9) (width 0.2) (layer "F.Cu") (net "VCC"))
 (segment (start 143.905 90.595) (end 142.59 91.91) (width 0.2) (layer "F.Cu") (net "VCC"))
 (segment (start 162.85 105.85) (end 163.5 106.5) (width 0.2) (layer "F.Cu") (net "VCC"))
 (segment (start 145.5375 90.595) (end 143.905 90.595) (width 0.2) (layer "F.Cu") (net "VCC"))
 (segment (start 159.445 90.595) (end 145.5375 90.595) (width 0.2) (layer "F.Cu") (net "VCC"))
 (segment (start 134.86 94.405) (end 124.5 104.765) (width 0.2) (layer "F.Cu") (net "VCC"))
 (segment (start 162.85 94) (end 159.445 90.595) (width 0.2) (layer "F.Cu") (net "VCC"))
 (segment (start 140.5575 94.5) (end 140.4625 94.405) (width 0.2) (layer "F.Cu") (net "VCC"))
 (segment (start 162.85 91.65) (end 162.85 94) (width 0.2) (layer "F.Cu") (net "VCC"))
 (segment (start 163 91.5) (end 162.85 91.65) (width 0.2) (layer "F.Cu") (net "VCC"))
 (segment (start 166.5 91.5) (end 163 91.5) (width 0.2) (layer "F.Cu") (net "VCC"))
 (segment (start 162.85 103) (end 162.85 105.85) (width 0.2) (layer "F.Cu") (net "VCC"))
 (segment (start 140.4625 94.405) (end 134.86 94.405) (width 0.2) (layer "F.Cu") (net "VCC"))
 (segment (start 163.5 106.5) (end 166.9 106.5) (width 0.2) (layer "F.Cu") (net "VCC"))
 (segment (start 142.59 91.91) (end 142.4 91.91) (width 0.2) (layer "F.Cu") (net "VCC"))
 (segment (start 142 94.5) (end 140.5575 94.5) (width 0.2) (layer "F.Cu") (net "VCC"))
 (via (at 142 94.5) (size 0.6) (drill 0.3) (layers "F.Cu" "B.Cu") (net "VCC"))
 (via (at 142.4 91.91) (size 0.6) (drill 0.3) (layers "F.Cu" "B.Cu") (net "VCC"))
 (segment (start 142 92.31) (end 142 94.5) (width 0.2) (layer "B.Cu") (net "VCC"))
 (segment (start 142.4 91.91) (end 142 92.31) (width 0.2) (layer "B.Cu") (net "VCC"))
 (segment (start 145.5375 94.405) (end 146.5 95.3675) (width 0.2) (layer "F.Cu") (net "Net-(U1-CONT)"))
 (segment (start 146.5 95.3675) (end 146.5 104) (width 0.2) (layer "F.Cu") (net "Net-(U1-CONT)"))
 (segment (start 164.5 96.85) (end 162.85 98.5) (width 0.2) (layer "F.Cu") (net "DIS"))
 (segment (start 162.85 98.5) (end 156.215 91.865) (width 0.2) (layer "F.Cu") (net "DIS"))
 (segment (start 164.5 94) (end 164.5 96.85) (width 0.2) (layer "F.Cu") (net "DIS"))
 (segment (start 156.215 91.865) (end 145.5375 91.865) (width 0.2) (layer "F.Cu") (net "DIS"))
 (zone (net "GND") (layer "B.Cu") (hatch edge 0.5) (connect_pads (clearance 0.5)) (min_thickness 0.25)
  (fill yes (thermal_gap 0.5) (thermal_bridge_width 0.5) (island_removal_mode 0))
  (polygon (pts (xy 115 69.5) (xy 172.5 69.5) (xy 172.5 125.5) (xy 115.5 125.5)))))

